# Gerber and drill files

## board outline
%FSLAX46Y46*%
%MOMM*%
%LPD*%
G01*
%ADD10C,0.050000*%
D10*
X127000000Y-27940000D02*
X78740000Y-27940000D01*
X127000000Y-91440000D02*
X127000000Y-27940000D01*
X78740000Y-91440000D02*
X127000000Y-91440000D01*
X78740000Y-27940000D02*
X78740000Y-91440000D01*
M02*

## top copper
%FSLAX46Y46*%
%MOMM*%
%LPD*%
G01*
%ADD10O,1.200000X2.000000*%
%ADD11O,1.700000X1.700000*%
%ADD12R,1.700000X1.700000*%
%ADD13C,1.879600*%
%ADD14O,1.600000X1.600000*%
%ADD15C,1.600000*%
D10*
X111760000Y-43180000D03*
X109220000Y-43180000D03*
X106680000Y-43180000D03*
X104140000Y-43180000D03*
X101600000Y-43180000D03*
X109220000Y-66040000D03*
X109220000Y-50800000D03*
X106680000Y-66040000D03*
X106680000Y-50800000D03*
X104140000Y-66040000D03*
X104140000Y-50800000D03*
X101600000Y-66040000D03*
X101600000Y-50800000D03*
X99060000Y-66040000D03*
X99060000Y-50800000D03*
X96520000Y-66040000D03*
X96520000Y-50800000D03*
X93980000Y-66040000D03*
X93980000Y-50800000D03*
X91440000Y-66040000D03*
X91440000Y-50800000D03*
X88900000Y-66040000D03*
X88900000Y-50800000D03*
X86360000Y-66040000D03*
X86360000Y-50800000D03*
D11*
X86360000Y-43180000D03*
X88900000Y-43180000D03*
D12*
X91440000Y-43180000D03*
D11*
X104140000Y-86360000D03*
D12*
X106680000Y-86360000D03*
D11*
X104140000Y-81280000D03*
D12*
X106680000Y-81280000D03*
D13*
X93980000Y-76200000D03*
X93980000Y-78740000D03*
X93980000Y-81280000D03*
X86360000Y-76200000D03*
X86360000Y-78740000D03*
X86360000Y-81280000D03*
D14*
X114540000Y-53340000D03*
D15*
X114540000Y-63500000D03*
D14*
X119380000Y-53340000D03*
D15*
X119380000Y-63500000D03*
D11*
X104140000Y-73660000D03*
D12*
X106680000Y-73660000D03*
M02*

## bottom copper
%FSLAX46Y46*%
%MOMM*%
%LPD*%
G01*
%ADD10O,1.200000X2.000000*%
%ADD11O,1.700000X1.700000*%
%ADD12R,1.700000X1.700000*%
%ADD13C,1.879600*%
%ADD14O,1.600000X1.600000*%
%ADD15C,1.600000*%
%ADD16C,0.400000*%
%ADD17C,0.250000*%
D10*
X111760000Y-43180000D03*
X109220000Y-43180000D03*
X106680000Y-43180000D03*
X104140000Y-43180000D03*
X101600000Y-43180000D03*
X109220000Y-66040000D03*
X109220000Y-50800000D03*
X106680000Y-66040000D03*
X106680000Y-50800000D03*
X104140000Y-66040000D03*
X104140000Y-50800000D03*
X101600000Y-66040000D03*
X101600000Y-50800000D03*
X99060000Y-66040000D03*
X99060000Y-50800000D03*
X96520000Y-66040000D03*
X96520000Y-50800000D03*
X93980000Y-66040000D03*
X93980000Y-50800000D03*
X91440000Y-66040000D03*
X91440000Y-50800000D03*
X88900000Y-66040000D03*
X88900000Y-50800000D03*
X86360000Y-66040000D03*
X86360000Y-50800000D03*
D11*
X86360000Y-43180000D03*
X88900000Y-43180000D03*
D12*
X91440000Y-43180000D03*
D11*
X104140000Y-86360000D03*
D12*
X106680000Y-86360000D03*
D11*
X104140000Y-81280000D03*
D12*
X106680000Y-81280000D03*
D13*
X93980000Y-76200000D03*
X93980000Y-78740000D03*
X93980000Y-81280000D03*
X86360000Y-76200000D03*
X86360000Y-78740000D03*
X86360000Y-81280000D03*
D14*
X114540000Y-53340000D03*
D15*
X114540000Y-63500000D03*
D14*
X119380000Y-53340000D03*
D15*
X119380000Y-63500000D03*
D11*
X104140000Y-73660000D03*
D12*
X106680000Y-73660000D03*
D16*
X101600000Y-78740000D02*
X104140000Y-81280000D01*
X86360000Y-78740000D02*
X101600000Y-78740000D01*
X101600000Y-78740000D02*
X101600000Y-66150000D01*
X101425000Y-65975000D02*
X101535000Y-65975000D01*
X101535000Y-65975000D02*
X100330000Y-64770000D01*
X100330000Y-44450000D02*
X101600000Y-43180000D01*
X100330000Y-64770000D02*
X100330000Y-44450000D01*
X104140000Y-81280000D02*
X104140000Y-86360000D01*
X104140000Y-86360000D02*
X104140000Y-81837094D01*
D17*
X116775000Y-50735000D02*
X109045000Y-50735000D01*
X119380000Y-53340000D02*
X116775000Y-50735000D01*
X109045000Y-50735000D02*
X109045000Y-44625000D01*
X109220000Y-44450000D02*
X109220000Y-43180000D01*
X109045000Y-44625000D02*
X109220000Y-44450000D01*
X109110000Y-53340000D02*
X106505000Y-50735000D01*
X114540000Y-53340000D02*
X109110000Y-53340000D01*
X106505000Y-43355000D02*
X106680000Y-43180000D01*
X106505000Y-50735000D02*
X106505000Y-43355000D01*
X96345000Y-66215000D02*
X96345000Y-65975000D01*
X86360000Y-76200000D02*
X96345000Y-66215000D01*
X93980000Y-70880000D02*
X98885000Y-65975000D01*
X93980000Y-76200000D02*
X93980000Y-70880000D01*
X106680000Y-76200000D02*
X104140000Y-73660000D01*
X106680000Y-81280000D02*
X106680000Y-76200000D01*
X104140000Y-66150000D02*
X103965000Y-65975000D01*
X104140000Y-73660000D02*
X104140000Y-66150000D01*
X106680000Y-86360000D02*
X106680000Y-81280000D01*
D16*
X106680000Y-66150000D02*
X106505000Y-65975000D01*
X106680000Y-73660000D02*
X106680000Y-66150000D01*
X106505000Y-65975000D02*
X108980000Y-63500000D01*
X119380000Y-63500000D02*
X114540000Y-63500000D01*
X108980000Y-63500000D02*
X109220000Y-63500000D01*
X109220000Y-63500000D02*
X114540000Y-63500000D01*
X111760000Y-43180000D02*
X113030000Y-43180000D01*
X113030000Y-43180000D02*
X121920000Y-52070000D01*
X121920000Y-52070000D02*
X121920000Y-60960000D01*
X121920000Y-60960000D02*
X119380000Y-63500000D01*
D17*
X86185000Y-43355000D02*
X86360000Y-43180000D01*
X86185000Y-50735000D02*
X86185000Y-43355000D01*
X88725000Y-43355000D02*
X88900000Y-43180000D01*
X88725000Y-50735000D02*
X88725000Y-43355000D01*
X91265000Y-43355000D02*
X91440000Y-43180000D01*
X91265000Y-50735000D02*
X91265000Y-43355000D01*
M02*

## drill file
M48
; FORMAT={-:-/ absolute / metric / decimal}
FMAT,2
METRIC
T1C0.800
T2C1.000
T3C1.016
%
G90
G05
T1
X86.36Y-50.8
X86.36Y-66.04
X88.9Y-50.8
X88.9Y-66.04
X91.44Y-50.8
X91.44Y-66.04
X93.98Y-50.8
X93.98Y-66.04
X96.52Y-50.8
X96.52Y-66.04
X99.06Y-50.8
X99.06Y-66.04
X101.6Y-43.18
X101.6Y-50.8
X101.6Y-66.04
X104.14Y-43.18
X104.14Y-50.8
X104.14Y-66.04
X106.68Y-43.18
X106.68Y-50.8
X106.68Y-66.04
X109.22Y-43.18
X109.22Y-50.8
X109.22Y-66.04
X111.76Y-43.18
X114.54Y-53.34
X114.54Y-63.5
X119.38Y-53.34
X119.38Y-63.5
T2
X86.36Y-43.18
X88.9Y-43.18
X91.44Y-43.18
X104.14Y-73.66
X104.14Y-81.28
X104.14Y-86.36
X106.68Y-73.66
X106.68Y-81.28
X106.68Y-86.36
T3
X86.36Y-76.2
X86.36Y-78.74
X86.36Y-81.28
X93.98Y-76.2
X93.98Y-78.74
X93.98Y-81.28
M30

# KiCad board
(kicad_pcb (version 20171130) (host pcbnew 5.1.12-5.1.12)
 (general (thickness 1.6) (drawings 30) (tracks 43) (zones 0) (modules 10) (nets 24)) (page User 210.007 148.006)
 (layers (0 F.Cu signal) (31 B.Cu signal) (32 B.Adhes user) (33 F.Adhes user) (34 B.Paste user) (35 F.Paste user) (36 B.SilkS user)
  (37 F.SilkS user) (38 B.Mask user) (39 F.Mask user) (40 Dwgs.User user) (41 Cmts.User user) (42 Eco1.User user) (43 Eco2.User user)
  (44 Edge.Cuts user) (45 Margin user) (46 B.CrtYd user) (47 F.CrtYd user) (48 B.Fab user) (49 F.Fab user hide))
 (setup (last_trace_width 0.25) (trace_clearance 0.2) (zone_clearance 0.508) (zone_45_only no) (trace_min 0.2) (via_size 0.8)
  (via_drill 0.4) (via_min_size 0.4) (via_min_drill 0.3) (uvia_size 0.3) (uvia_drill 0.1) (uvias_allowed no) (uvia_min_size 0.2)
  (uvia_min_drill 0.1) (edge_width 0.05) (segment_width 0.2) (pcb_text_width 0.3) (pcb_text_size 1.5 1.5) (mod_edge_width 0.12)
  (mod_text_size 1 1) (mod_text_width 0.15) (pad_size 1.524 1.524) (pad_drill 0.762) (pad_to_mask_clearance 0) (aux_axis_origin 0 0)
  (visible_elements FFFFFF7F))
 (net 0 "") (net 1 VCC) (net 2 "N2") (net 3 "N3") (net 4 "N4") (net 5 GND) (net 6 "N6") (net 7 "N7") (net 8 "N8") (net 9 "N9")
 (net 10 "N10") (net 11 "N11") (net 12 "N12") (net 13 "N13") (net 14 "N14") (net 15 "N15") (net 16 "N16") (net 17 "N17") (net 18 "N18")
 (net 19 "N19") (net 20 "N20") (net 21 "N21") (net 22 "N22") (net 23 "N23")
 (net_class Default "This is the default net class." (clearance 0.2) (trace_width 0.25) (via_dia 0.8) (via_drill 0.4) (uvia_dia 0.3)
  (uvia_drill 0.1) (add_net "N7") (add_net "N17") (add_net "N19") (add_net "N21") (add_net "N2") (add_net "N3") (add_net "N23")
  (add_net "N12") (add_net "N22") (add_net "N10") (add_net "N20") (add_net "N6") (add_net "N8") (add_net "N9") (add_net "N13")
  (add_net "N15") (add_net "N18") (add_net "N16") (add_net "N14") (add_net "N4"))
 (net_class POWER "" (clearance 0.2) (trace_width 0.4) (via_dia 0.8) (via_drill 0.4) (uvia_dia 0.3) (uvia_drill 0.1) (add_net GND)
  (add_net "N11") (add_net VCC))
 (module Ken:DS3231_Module (layer F.Cu) (at 106.68 43.18)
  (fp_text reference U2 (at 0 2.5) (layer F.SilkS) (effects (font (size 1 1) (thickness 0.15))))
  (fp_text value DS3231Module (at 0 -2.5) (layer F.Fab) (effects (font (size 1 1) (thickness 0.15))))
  (pad 5 thru_hole oval (at 5.08 0) (size 1.2 2) (drill 0.8) (layers *.Cu *.Mask) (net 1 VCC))
  (pad 4 thru_hole oval (at 2.54 0) (size 1.2 2) (drill 0.8) (layers *.Cu *.Mask) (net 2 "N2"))
  (pad 3 thru_hole oval (at 0 0) (size 1.2 2) (drill 0.8) (layers *.Cu *.Mask) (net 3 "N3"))
  (pad 2 thru_hole oval (at -2.54 0) (size 1.2 2) (drill 0.8) (layers *.Cu *.Mask) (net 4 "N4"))
  (pad 1 thru_hole oval (at -5.08 0) (size 1.2 2) (drill 0.8) (layers *.Cu *.Mask) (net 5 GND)))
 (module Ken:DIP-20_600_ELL (layer F.Cu) (at 97.79 58.42)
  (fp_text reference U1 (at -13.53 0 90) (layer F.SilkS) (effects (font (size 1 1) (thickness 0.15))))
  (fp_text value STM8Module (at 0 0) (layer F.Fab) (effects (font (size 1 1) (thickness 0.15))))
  (pad 10 thru_hole oval (at 11.43 7.62) (size 1.2 2) (drill 0.8) (layers *.Cu *.Mask) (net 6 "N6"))
  (pad 11 thru_hole oval (at 11.43 -7.62) (size 1.2 2) (drill 0.8) (layers *.Cu *.Mask) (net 2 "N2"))
  (pad 9 thru_hole oval (at 8.89 7.62) (size 1.2 2) (drill 0.8) (layers *.Cu *.Mask) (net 1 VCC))
  (pad 12 thru_hole oval (at 8.89 -7.62) (size 1.2 2) (drill 0.8) (layers *.Cu *.Mask) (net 3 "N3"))
  (pad 8 thru_hole oval (at 6.35 7.62) (size 1.2 2) (drill 0.8) (layers *.Cu *.Mask) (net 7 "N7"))
  (pad 13 thru_hole oval (at 6.35 -7.62) (size 1.2 2) (drill 0.8) (layers *.Cu *.Mask) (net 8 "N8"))
  (pad 7 thru_hole oval (at 3.81 7.62) (size 1.2 2) (drill 0.8) (layers *.Cu *.Mask) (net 5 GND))
  (pad 14 thru_hole oval (at 3.81 -7.62) (size 1.2 2) (drill 0.8) (layers *.Cu *.Mask) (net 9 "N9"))
  (pad 6 thru_hole oval (at 1.27 7.62) (size 1.2 2) (drill 0.8) (layers *.Cu *.Mask) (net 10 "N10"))
  (pad 15 thru_hole oval (at 1.27 -7.62) (size 1.2 2) (drill 0.8) (layers *.Cu *.Mask) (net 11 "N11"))
  (pad 5 thru_hole oval (at -1.27 7.62) (size 1.2 2) (drill 0.8) (layers *.Cu *.Mask) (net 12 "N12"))
  (pad 16 thru_hole oval (at -1.27 -7.62) (size 1.2 2) (drill 0.8) (layers *.Cu *.Mask) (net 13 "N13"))
  (pad 4 thru_hole oval (at -3.81 7.62) (size 1.2 2) (drill 0.8) (layers *.Cu *.Mask) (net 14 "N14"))
  (pad 17 thru_hole oval (at -3.81 -7.62) (size 1.2 2) (drill 0.8) (layers *.Cu *.Mask) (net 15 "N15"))
  (pad 3 thru_hole oval (at -6.35 7.62) (size 1.2 2) (drill 0.8) (layers *.Cu *.Mask) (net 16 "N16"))
  (pad 18 thru_hole oval (at -6.35 -7.62) (size 1.2 2) (drill 0.8) (layers *.Cu *.Mask) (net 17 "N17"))
  (pad 2 thru_hole oval (at -8.89 7.62) (size 1.2 2) (drill 0.8) (layers *.Cu *.Mask) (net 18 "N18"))
  (pad 19 thru_hole oval (at -8.89 -7.62) (size 1.2 2) (drill 0.8) (layers *.Cu *.Mask) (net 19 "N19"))
  (pad 1 thru_hole oval (at -11.43 7.62) (size 1.2 2) (drill 0.8) (layers *.Cu *.Mask) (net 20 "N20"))
  (pad 20 thru_hole oval (at -11.43 -7.62) (size 1.2 2) (drill 0.8) (layers *.Cu *.Mask) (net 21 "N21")))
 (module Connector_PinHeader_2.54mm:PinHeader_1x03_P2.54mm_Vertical (layer F.Cu) (at 91.44 43.18 270)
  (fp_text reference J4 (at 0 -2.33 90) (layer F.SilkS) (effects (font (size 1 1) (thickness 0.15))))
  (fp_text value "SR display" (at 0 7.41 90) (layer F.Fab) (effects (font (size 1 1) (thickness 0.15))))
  (pad 3 thru_hole oval (at 0 5.08 270) (size 1.7 1.7) (drill 1) (layers *.Cu *.Mask) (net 21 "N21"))
  (pad 2 thru_hole oval (at 0 2.54 270) (size 1.7 1.7) (drill 1) (layers *.Cu *.Mask) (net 19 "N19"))
  (pad 1 thru_hole rect (at 0 0 270) (size 1.7 1.7) (drill 1) (layers *.Cu *.Mask) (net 17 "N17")))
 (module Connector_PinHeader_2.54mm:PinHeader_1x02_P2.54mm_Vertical (layer F.Cu) (at 106.68 86.36 270)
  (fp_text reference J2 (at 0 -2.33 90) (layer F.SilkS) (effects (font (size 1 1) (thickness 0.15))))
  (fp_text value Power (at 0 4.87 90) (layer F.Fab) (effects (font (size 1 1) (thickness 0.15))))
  (pad 2 thru_hole oval (at 0 2.54 270) (size 1.7 1.7) (drill 1) (layers *.Cu *.Mask) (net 5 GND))
  (pad 1 thru_hole rect (at 0 0 270) (size 1.7 1.7) (drill 1) (layers *.Cu *.Mask) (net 7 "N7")))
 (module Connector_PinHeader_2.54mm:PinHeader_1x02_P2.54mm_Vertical (layer F.Cu) (at 106.68 81.28 270)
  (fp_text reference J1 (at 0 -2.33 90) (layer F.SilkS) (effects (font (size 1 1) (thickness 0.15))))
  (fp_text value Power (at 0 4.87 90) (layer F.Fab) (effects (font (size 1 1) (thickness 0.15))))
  (pad 2 thru_hole oval (at 0 2.54 270) (size 1.7 1.7) (drill 1) (layers *.Cu *.Mask) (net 5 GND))
  (pad 1 thru_hole rect (at 0 0 270) (size 1.7 1.7) (drill 1) (layers *.Cu *.Mask) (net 7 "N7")))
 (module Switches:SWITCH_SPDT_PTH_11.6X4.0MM (layer F.Cu) (at 93.98 78.74 180)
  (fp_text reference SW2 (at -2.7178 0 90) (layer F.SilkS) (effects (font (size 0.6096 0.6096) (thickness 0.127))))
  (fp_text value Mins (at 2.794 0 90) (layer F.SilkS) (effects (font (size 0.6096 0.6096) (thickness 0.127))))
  (pad 3 thru_hole circle (at 0 2.54 180) (size 1.8796 1.8796) (drill 1.016) (layers *.Cu *.Mask) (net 10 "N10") (solder_mask_margin 0.1016))
  (pad 2 thru_hole circle (at 0 0 180) (size 1.8796 1.8796) (drill 1.016) (layers *.Cu *.Mask) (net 5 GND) (solder_mask_margin 0.1016))
  (pad 1 thru_hole circle (at 0 -2.54 180) (size 1.8796 1.8796) (drill 1.016) (layers *.Cu *.Mask) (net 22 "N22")
   (solder_mask_margin 0.1016)))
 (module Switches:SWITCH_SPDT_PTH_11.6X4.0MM (layer F.Cu) (at 86.36 78.74 180)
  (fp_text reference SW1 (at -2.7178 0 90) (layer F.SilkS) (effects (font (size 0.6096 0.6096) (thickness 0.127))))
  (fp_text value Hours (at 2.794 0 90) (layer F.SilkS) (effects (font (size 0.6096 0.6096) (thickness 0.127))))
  (pad 3 thru_hole circle (at 0 2.54 180) (size 1.8796 1.8796) (drill 1.016) (layers *.Cu *.Mask) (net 12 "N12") (solder_mask_margin 0.1016))
  (pad 2 thru_hole circle (at 0 0 180) (size 1.8796 1.8796) (drill 1.016) (layers *.Cu *.Mask) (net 5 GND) (solder_mask_margin 0.1016))
  (pad 1 thru_hole circle (at 0 -2.54 180) (size 1.8796 1.8796) (drill 1.016) (layers *.Cu *.Mask) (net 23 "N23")
   (solder_mask_margin 0.1016)))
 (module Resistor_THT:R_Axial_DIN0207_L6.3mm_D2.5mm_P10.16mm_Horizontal (layer F.Cu) (at 114.54 63.5 90)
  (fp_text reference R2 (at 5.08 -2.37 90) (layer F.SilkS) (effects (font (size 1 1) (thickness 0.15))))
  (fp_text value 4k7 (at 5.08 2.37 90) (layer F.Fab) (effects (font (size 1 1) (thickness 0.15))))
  (pad 2 thru_hole oval (at 10.16 0 90) (size 1.6 1.6) (drill 0.8) (layers *.Cu *.Mask) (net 3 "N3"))
  (pad 1 thru_hole circle (at 0 0 90) (size 1.6 1.6) (drill 0.8) (layers *.Cu *.Mask) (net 1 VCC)))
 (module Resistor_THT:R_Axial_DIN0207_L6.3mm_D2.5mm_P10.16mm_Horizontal (layer F.Cu) (at 119.38 63.5 90)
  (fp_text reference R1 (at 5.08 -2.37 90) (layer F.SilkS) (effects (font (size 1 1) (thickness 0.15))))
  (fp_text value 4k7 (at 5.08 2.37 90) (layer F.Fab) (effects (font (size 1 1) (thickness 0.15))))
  (pad 2 thru_hole oval (at 10.16 0 90) (size 1.6 1.6) (drill 0.8) (layers *.Cu *.Mask) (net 2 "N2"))
  (pad 1 thru_hole circle (at 0 0 90) (size 1.6 1.6) (drill 0.8) (layers *.Cu *.Mask) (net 1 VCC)))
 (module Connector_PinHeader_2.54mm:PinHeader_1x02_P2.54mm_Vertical (layer F.Cu) (at 106.68 73.66 270)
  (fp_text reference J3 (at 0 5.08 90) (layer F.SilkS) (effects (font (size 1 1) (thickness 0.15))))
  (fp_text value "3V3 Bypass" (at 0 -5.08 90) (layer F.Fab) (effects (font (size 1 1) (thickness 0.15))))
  (pad 2 thru_hole oval (at 0 2.54 270) (size 1.7 1.7) (drill 1) (layers *.Cu *.Mask) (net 7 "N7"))
  (pad 1 thru_hole rect (at 0 0 270) (size 1.7 1.7) (drill 1) (layers *.Cu *.Mask) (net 1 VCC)))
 (gr_line (start 127 27.94) (end 78.74 27.94) (layer Edge.Cuts) (width 0.05))
 (gr_line (start 127 91.44) (end 127 27.94) (layer Edge.Cuts) (width 0.05))
 (gr_line (start 78.74 91.44) (end 127 91.44) (layer Edge.Cuts) (width 0.05))
 (gr_line (start 78.74 27.94) (end 78.74 91.44) (layer Edge.Cuts) (width 0.05))
 (segment (start 101.6 78.74) (end 104.14 81.28) (width 0.4) (layer B.Cu) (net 5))
 (segment (start 86.36 78.74) (end 101.6 78.74) (width 0.4) (layer B.Cu) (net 5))
 (segment (start 101.6 78.74) (end 101.6 66.15) (width 0.4) (layer B.Cu) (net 5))
 (segment (start 101.425 65.975) (end 101.535 65.975) (width 0.4) (layer B.Cu) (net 5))
 (segment (start 101.535 65.975) (end 100.33 64.77) (width 0.4) (layer B.Cu) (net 5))
 (segment (start 100.33 44.45) (end 101.6 43.18) (width 0.4) (layer B.Cu) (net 5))
 (segment (start 100.33 64.77) (end 100.33 44.45) (width 0.4) (layer B.Cu) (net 5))
 (segment (start 104.14 81.28) (end 104.14 86.36) (width 0.4) (layer B.Cu) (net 5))
 (segment (start 104.14 86.36) (end 104.14 81.837094) (width 0.4) (layer B.Cu) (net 5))
 (segment (start 116.775 50.735) (end 109.045 50.735) (width 0.25) (layer B.Cu) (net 2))
 (segment (start 119.38 53.34) (end 116.775 50.735) (width 0.25) (layer B.Cu) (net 2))
 (segment (start 109.045 50.735) (end 109.045 44.625) (width 0.25) (layer B.Cu) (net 2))
 (segment (start 109.22 44.45) (end 109.22 43.18) (width 0.25) (layer B.Cu) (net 2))
 (segment (start 109.045 44.625) (end 109.22 44.45) (width 0.25) (layer B.Cu) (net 2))
 (segment (start 109.11 53.34) (end 106.505 50.735) (width 0.25) (layer B.Cu) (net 3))
 (segment (start 114.54 53.34) (end 109.11 53.34) (width 0.25) (layer B.Cu) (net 3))
 (segment (start 106.505 43.355) (end 106.68 43.18) (width 0.25) (layer B.Cu) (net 3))
 (segment (start 106.505 50.735) (end 106.505 43.355) (width 0.25) (layer B.Cu) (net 3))
 (segment (start 96.345 66.215) (end 96.345 65.975) (width 0.25) (layer B.Cu) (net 12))
 (segment (start 86.36 76.2) (end 96.345 66.215) (width 0.25) (layer B.Cu) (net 12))
 (segment (start 93.98 70.88) (end 98.885 65.975) (width 0.25) (layer B.Cu) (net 10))
 (segment (start 93.98 76.2) (end 93.98 70.88) (width 0.25) (layer B.Cu) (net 10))
 (segment (start 106.68 76.2) (end 104.14 73.66) (width 0.25) (layer B.Cu) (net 7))
 (segment (start 106.68 81.28) (end 106.68 76.2) (width 0.25) (layer B.Cu) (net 7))
 (segment (start 104.14 66.15) (end 103.965 65.975) (width 0.25) (layer B.Cu) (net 7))
 (segment (start 104.14 73.66) (end 104.14 66.15) (width 0.25) (layer B.Cu) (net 7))
 (segment (start 106.68 86.36) (end 106.68 81.28) (width 0.25) (layer B.Cu) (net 7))
 (segment (start 106.68 66.15) (end 106.505 65.975) (width 0.4) (layer B.Cu) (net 1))
 (segment (start 106.68 73.66) (end 106.68 66.15) (width 0.4) (layer B.Cu) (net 1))
 (segment (start 106.505 65.975) (end 108.98 63.5) (width 0.4) (layer B.Cu) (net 1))
 (segment (start 119.38 63.5) (end 114.54 63.5) (width 0.4) (layer B.Cu) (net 1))
 (segment (start 108.98 63.5) (end 109.22 63.5) (width 0.4) (layer B.Cu) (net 1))
 (segment (start 109.22 63.5) (end 114.54 63.5) (width 0.4) (layer B.Cu) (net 1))
 (segment (start 111.76 43.18) (end 113.03 43.18) (width 0.4) (layer B.Cu) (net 1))
 (segment (start 113.03 43.18) (end 121.92 52.07) (width 0.4) (layer B.Cu) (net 1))
 (segment (start 121.92 52.07) (end 121.92 60.96) (width 0.4) (layer B.Cu) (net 1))
 (segment (start 121.92 60.96) (end 119.38 63.5) (width 0.4) (layer B.Cu) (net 1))
 (segment (start 86.185 43.355) (end 86.36 43.18) (width 0.25) (layer B.Cu) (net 21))
 (segment (start 86.185 50.735) (end 86.185 43.355) (width 0.25) (layer B.Cu) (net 21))
 (segment (start 88.725 43.355) (end 88.9 43.18) (width 0.25) (layer B.Cu) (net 19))
 (segment (start 88.725 50.735) (end 88.725 43.355) (width 0.25) (layer B.Cu) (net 19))
 (segment (start 91.265 43.355) (end 91.44 43.18) (width 0.25) (layer B.Cu) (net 17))
 (segment (start 91.265 50.735) (end 91.265 43.355) (width 0.25) (layer B.Cu) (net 17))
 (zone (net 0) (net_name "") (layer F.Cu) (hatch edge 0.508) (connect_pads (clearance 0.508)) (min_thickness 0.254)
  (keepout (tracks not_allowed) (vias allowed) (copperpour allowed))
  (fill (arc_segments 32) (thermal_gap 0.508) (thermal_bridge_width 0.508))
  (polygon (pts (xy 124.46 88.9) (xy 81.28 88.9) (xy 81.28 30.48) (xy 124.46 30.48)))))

